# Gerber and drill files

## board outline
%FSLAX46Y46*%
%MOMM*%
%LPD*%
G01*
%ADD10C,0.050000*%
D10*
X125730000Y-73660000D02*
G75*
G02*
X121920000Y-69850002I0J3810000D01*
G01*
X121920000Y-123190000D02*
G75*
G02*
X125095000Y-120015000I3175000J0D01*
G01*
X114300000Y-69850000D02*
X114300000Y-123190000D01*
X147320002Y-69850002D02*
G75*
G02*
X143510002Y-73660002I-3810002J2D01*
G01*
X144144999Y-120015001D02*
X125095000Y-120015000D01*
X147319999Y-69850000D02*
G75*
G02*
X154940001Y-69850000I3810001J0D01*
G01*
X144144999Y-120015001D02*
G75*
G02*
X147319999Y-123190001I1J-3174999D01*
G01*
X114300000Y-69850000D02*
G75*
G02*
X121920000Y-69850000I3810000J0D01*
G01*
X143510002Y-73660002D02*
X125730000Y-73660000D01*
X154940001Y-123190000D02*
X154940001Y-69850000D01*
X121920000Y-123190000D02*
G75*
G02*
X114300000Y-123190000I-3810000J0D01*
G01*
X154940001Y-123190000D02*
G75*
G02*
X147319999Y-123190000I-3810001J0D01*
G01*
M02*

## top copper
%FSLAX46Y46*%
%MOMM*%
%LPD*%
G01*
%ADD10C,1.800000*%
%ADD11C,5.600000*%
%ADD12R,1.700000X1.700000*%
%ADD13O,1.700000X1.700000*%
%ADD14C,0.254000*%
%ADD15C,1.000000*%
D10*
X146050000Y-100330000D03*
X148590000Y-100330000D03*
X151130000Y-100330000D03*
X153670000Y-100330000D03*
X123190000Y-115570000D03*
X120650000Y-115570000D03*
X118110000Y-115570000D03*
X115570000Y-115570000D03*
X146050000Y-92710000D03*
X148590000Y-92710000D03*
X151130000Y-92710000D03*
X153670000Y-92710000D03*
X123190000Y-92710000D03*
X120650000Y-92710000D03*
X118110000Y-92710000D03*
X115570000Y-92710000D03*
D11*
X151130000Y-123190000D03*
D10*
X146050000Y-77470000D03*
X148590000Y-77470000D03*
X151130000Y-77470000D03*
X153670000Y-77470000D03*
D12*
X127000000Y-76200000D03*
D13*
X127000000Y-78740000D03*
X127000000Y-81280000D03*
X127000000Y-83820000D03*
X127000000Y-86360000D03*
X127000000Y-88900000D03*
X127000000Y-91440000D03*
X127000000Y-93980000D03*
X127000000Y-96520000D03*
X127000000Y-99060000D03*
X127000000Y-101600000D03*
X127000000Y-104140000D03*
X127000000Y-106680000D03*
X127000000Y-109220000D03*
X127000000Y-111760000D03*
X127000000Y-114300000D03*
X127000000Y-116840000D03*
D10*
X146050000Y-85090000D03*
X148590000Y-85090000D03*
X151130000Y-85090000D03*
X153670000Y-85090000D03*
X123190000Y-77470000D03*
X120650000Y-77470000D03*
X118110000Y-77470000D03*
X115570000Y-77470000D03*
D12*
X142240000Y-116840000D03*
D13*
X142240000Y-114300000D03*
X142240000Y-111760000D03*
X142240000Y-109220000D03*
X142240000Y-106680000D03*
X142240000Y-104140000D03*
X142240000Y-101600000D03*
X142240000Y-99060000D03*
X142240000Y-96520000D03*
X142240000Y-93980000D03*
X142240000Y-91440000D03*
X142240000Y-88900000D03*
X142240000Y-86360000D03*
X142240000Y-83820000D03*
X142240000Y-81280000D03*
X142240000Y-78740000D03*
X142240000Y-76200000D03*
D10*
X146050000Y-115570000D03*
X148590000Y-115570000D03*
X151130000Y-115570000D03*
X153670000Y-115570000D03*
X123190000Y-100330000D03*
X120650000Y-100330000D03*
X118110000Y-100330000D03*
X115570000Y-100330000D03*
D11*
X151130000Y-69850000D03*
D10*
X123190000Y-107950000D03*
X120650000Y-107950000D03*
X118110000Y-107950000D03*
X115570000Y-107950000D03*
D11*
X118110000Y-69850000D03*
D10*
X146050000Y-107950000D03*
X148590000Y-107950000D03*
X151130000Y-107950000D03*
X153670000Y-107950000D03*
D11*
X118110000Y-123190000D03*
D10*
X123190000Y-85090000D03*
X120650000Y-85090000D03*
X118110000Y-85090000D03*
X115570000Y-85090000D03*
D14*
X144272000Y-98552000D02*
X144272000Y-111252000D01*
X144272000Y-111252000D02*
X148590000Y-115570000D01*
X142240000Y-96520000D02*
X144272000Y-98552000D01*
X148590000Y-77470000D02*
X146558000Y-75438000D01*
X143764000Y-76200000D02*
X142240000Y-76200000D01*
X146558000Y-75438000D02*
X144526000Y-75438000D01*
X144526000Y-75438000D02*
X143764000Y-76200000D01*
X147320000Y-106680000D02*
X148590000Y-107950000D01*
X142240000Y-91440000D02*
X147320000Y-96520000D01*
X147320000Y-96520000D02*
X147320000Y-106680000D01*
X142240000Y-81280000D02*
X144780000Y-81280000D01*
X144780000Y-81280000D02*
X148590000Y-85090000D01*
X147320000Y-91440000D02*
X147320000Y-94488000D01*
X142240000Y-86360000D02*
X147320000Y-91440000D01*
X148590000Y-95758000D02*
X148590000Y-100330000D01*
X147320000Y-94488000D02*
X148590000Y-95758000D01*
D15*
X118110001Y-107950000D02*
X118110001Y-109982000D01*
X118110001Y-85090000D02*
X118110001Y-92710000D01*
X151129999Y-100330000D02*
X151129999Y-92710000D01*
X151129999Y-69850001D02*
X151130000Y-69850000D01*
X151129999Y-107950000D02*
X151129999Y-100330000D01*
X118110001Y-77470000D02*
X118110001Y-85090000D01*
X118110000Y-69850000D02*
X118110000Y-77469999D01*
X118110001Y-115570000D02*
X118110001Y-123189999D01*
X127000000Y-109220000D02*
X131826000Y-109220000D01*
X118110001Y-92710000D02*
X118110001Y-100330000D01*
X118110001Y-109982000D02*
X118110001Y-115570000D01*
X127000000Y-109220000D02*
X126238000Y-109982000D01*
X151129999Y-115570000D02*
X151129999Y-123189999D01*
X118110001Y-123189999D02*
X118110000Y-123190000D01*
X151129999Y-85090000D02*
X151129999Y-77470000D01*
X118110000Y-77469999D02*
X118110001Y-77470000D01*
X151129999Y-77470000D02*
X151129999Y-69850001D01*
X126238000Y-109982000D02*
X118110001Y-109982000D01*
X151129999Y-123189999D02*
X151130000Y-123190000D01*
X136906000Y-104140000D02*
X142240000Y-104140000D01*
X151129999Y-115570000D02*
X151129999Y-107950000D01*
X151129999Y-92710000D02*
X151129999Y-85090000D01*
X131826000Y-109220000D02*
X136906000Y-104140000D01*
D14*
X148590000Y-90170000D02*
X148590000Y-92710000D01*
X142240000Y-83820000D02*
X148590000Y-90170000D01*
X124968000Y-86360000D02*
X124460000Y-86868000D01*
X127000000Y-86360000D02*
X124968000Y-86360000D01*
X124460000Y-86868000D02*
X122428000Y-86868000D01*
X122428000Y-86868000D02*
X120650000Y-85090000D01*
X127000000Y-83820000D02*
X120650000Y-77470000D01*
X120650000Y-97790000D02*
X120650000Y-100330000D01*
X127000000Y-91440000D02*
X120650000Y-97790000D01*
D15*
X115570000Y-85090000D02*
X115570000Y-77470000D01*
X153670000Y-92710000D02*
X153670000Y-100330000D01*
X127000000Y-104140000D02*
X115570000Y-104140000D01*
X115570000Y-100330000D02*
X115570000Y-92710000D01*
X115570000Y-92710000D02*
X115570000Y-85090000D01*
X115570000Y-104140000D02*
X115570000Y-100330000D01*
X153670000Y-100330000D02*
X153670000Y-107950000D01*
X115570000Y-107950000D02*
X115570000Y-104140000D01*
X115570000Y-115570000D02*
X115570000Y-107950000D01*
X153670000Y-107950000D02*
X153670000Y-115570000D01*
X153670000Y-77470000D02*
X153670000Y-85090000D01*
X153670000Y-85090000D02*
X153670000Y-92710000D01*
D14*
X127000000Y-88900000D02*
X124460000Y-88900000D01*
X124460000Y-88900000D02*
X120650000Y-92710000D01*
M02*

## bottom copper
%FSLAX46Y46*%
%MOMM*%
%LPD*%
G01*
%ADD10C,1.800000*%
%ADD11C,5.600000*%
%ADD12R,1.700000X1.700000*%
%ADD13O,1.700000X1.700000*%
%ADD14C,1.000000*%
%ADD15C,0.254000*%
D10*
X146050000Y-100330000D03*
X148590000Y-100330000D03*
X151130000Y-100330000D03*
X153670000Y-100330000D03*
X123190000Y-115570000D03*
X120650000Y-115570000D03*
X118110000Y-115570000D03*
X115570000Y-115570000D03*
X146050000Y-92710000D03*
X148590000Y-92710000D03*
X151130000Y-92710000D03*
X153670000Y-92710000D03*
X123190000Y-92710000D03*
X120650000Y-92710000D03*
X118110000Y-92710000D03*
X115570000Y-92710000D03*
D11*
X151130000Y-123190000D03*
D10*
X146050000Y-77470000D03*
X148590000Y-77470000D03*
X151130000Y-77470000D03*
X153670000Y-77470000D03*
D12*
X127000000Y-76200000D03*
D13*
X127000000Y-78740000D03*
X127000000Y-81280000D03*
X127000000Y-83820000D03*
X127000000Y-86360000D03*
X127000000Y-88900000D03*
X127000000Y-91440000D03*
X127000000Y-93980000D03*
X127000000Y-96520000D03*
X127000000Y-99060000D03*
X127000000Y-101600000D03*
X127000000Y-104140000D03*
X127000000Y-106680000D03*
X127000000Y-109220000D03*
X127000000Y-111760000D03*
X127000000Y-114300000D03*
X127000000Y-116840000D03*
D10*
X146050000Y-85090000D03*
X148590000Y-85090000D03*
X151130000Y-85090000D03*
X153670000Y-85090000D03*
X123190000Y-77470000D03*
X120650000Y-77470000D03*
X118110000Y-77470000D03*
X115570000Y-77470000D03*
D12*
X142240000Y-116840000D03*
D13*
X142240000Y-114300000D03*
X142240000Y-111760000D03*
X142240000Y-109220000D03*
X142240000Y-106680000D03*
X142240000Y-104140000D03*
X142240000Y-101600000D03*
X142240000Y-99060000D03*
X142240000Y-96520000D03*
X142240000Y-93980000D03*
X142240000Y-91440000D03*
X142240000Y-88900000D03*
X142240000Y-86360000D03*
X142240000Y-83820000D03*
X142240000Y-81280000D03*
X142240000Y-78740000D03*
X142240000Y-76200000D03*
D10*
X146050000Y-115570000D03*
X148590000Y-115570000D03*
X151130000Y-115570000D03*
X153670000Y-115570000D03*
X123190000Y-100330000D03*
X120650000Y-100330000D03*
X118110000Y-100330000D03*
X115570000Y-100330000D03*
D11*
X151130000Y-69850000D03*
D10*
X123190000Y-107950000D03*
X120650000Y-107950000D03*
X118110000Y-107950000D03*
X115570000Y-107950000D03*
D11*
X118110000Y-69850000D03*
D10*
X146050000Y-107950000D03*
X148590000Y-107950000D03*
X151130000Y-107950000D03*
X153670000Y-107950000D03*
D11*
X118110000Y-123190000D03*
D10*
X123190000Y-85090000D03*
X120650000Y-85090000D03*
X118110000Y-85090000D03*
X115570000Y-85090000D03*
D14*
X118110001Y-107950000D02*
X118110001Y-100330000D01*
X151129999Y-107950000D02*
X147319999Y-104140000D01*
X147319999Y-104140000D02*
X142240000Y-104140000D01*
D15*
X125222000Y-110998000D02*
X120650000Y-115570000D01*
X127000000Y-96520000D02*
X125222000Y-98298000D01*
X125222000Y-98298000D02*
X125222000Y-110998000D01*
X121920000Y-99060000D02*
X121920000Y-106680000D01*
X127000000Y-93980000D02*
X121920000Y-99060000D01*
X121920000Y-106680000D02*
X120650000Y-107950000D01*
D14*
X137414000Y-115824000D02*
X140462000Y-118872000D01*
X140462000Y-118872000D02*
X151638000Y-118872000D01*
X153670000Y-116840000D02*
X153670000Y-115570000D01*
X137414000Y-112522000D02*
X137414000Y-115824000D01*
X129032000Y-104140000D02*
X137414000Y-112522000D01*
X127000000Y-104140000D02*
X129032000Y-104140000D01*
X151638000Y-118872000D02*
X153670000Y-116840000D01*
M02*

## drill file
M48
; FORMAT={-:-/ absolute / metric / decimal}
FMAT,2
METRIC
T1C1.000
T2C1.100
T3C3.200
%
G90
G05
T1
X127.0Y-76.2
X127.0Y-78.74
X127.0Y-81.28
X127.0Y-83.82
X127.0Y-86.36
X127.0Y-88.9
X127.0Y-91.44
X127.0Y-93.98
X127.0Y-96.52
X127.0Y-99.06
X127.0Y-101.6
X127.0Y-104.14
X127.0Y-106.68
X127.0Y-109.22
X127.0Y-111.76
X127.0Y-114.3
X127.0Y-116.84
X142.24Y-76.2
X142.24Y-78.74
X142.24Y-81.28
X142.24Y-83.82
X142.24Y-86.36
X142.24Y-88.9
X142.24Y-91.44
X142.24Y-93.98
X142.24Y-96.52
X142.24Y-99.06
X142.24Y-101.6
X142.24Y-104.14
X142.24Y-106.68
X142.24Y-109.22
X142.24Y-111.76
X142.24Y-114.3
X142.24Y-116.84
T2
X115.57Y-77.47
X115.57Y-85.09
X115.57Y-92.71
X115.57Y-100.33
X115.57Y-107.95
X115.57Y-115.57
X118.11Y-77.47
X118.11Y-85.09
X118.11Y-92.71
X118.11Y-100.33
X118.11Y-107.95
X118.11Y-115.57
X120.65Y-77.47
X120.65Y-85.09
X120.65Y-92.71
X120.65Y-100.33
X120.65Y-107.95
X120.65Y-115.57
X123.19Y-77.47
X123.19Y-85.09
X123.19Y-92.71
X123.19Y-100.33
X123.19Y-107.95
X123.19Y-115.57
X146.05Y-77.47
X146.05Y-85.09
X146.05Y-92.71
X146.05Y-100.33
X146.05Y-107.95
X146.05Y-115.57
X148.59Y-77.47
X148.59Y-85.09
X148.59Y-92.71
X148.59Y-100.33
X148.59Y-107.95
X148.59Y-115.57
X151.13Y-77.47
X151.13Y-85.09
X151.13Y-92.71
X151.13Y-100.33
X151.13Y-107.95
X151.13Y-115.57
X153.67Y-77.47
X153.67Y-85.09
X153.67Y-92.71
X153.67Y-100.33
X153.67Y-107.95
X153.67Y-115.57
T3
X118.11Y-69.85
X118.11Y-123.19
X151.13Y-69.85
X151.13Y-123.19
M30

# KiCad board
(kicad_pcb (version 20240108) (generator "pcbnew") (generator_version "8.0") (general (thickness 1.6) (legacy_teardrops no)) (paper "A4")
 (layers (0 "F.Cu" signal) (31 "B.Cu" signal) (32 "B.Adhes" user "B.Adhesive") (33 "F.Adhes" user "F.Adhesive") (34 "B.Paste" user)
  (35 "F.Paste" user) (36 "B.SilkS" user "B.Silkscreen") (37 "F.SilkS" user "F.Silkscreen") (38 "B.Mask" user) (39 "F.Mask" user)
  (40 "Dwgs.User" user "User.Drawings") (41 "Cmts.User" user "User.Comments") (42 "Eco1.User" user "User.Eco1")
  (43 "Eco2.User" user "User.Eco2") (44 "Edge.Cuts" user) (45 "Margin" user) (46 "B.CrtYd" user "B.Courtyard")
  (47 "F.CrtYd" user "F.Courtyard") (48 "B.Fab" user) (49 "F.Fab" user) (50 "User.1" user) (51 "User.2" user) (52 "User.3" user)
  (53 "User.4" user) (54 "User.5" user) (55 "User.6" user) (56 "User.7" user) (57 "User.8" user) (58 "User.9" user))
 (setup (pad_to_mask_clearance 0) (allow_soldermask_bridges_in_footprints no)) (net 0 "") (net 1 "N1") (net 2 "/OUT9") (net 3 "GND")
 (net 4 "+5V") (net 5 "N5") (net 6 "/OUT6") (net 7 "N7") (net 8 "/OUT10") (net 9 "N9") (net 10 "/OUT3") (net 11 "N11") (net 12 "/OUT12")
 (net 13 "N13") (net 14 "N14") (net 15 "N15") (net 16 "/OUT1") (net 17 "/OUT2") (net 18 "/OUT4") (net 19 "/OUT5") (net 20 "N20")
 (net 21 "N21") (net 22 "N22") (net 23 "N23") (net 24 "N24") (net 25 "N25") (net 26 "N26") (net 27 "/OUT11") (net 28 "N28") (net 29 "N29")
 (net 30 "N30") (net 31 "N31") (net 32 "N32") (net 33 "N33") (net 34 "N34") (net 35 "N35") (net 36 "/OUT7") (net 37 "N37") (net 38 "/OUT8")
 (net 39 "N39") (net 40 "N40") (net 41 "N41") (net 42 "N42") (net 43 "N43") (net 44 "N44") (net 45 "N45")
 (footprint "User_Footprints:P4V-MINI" (layer "F.Cu") (at 146.05 100.33)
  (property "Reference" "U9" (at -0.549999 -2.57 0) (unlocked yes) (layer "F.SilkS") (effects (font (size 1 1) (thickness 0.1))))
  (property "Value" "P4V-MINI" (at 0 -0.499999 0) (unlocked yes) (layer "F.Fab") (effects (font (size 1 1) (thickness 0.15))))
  (pad "1" thru_hole circle (at 0 0) (size 1.8 1.8) (drill 1.1) (layers "*.Cu" "*.Mask") (remove_unused_layers no) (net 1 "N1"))
  (pad "2" thru_hole circle (at 2.54 0) (size 1.8 1.8) (drill 1.1) (layers "*.Cu" "*.Mask") (remove_unused_layers no) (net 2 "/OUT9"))
  (pad "3" thru_hole circle (at 5.08 0) (size 1.8 1.8) (drill 1.1) (layers "*.Cu" "*.Mask") (remove_unused_layers no) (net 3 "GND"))
  (pad "4" thru_hole circle (at 7.62 0) (size 1.8 1.8) (drill 1.1) (layers "*.Cu" "*.Mask") (remove_unused_layers no) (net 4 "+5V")))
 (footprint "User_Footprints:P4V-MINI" (layer "F.Cu") (at 123.19 115.57 180)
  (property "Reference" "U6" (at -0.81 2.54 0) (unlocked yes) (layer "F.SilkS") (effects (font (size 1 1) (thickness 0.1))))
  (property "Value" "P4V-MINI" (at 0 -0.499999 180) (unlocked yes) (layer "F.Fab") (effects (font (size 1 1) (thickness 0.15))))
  (pad "1" thru_hole circle (at 0 0 180) (size 1.8 1.8) (drill 1.1) (layers "*.Cu" "*.Mask") (remove_unused_layers no) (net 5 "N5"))
  (pad "2" thru_hole circle (at 2.54 0 180) (size 1.8 1.8) (drill 1.1) (layers "*.Cu" "*.Mask") (remove_unused_layers no) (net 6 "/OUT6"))
  (pad "3" thru_hole circle (at 5.08 0 180) (size 1.8 1.8) (drill 1.1) (layers "*.Cu" "*.Mask") (remove_unused_layers no) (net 3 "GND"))
  (pad "4" thru_hole circle (at 7.62 0 180) (size 1.8 1.8) (drill 1.1) (layers "*.Cu" "*.Mask") (remove_unused_layers no) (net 4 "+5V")))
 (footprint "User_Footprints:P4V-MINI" (layer "F.Cu") (at 146.05 92.71)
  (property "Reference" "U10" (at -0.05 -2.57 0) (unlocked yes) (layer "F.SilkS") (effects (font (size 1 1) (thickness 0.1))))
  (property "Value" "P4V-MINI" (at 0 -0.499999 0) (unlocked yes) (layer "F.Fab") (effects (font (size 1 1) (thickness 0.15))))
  (pad "1" thru_hole circle (at 0 0) (size 1.8 1.8) (drill 1.1) (layers "*.Cu" "*.Mask") (remove_unused_layers no) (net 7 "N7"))
  (pad "2" thru_hole circle (at 2.54 0) (size 1.8 1.8) (drill 1.1) (layers "*.Cu" "*.Mask") (remove_unused_layers no) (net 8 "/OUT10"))
  (pad "3" thru_hole circle (at 5.08 0) (size 1.8 1.8) (drill 1.1) (layers "*.Cu" "*.Mask") (remove_unused_layers no) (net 3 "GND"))
  (pad "4" thru_hole circle (at 7.62 0) (size 1.8 1.8) (drill 1.1) (layers "*.Cu" "*.Mask") (remove_unused_layers no) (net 4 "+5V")))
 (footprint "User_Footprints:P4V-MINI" (layer "F.Cu") (at 123.19 92.71 180)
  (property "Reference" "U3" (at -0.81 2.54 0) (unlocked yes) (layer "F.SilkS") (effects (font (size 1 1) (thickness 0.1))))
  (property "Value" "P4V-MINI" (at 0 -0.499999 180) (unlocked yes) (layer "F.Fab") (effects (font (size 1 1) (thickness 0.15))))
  (pad "1" thru_hole circle (at 0 0 180) (size 1.8 1.8) (drill 1.1) (layers "*.Cu" "*.Mask") (remove_unused_layers no) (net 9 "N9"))
  (pad "2" thru_hole circle (at 2.54 0 180) (size 1.8 1.8) (drill 1.1) (layers "*.Cu" "*.Mask") (remove_unused_layers no) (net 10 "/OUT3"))
  (pad "3" thru_hole circle (at 5.08 0 180) (size 1.8 1.8) (drill 1.1) (layers "*.Cu" "*.Mask") (remove_unused_layers no) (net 3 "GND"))
  (pad "4" thru_hole circle (at 7.62 0 180) (size 1.8 1.8) (drill 1.1) (layers "*.Cu" "*.Mask") (remove_unused_layers no) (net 4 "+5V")))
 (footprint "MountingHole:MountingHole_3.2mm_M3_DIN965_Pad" (layer "F.Cu") (at 151.13 123.19)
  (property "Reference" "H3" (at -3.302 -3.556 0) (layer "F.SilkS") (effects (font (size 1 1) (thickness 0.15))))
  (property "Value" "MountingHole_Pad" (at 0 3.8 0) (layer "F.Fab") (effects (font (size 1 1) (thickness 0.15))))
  (pad "1" thru_hole circle (at 0 0) (size 5.6 5.6) (drill 3.2) (layers "*.Cu" "*.Mask") (remove_unused_layers no) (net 3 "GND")))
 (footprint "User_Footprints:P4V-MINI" (layer "F.Cu") (at 146.05 77.47)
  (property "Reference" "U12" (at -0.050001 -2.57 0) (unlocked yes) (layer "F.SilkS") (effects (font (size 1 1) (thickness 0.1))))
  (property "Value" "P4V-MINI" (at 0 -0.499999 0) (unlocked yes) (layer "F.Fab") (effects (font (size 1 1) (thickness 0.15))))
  (pad "1" thru_hole circle (at 0 0) (size 1.8 1.8) (drill 1.1) (layers "*.Cu" "*.Mask") (remove_unused_layers no) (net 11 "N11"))
  (pad "2" thru_hole circle (at 2.54 0) (size 1.8 1.8) (drill 1.1) (layers "*.Cu" "*.Mask") (remove_unused_layers no) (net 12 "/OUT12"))
  (pad "3" thru_hole circle (at 5.08 0) (size 1.8 1.8) (drill 1.1) (layers "*.Cu" "*.Mask") (remove_unused_layers no) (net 3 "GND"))
  (pad "4" thru_hole circle (at 7.62 0) (size 1.8 1.8) (drill 1.1) (layers "*.Cu" "*.Mask") (remove_unused_layers no) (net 4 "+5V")))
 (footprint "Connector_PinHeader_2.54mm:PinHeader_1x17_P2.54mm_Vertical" (layer "F.Cu") (at 127 76.2)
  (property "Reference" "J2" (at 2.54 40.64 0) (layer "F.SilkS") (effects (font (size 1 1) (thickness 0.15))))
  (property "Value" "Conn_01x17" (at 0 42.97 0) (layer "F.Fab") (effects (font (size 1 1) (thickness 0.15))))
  (pad "1" thru_hole rect (at 0 0) (size 1.7 1.7) (drill 1) (layers "*.Cu" "*.Mask") (remove_unused_layers no) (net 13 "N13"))
  (pad "2" thru_hole oval (at 0 2.54) (size 1.7 1.7) (drill 1) (layers "*.Cu" "*.Mask") (remove_unused_layers no) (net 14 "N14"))
  (pad "3" thru_hole oval (at 0 5.08) (size 1.7 1.7) (drill 1) (layers "*.Cu" "*.Mask") (remove_unused_layers no) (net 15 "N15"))
  (pad "4" thru_hole oval (at 0 7.62) (size 1.7 1.7) (drill 1) (layers "*.Cu" "*.Mask") (remove_unused_layers no) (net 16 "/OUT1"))
  (pad "5" thru_hole oval (at 0 10.16) (size 1.7 1.7) (drill 1) (layers "*.Cu" "*.Mask") (remove_unused_layers no) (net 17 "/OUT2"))
  (pad "6" thru_hole oval (at 0 12.7) (size 1.7 1.7) (drill 1) (layers "*.Cu" "*.Mask") (remove_unused_layers no) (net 10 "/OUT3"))
  (pad "7" thru_hole oval (at 0 15.24) (size 1.7 1.7) (drill 1) (layers "*.Cu" "*.Mask") (remove_unused_layers no) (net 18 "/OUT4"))
  (pad "8" thru_hole oval (at 0 17.78) (size 1.7 1.7) (drill 1) (layers "*.Cu" "*.Mask") (remove_unused_layers no) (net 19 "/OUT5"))
  (pad "9" thru_hole oval (at 0 20.32) (size 1.7 1.7) (drill 1) (layers "*.Cu" "*.Mask") (remove_unused_layers no) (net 6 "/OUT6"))
  (pad "10" thru_hole oval (at 0 22.86) (size 1.7 1.7) (drill 1) (layers "*.Cu" "*.Mask") (remove_unused_layers no) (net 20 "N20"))
  (pad "11" thru_hole oval (at 0 25.4) (size 1.7 1.7) (drill 1) (layers "*.Cu" "*.Mask") (remove_unused_layers no) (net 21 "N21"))
  (pad "12" thru_hole oval (at 0 27.94) (size 1.7 1.7) (drill 1) (layers "*.Cu" "*.Mask") (remove_unused_layers no) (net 4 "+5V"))
  (pad "13" thru_hole oval (at 0 30.48) (size 1.7 1.7) (drill 1) (layers "*.Cu" "*.Mask") (remove_unused_layers no) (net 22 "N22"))
  (pad "14" thru_hole oval (at 0 33.02) (size 1.7 1.7) (drill 1) (layers "*.Cu" "*.Mask") (remove_unused_layers no) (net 3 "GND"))
  (pad "15" thru_hole oval (at 0 35.56) (size 1.7 1.7) (drill 1) (layers "*.Cu" "*.Mask") (remove_unused_layers no) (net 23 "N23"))
  (pad "16" thru_hole oval (at 0 38.1) (size 1.7 1.7) (drill 1) (layers "*.Cu" "*.Mask") (remove_unused_layers no) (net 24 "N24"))
  (pad "17" thru_hole oval (at 0 40.64) (size 1.7 1.7) (drill 1) (layers "*.Cu" "*.Mask") (remove_unused_layers no) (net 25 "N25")))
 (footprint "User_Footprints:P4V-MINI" (layer "F.Cu") (at 146.05 85.09)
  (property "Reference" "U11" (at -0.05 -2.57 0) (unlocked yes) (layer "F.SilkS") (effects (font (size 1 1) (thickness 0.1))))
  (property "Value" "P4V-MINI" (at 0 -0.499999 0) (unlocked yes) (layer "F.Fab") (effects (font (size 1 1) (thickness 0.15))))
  (pad "1" thru_hole circle (at 0 0) (size 1.8 1.8) (drill 1.1) (layers "*.Cu" "*.Mask") (remove_unused_layers no) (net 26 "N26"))
  (pad "2" thru_hole circle (at 2.54 0) (size 1.8 1.8) (drill 1.1) (layers "*.Cu" "*.Mask") (remove_unused_layers no) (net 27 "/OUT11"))
  (pad "3" thru_hole circle (at 5.08 0) (size 1.8 1.8) (drill 1.1) (layers "*.Cu" "*.Mask") (remove_unused_layers no) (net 3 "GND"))
  (pad "4" thru_hole circle (at 7.62 0) (size 1.8 1.8) (drill 1.1) (layers "*.Cu" "*.Mask") (remove_unused_layers no) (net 4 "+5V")))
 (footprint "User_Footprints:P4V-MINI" (layer "F.Cu") (at 123.19 77.47 180)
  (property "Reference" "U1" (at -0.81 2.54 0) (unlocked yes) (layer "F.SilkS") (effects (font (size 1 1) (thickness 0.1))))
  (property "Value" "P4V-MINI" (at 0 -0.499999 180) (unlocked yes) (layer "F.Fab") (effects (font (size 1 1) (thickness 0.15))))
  (pad "1" thru_hole circle (at 0 0 180) (size 1.8 1.8) (drill 1.1) (layers "*.Cu" "*.Mask") (remove_unused_layers no) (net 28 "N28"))
  (pad "2" thru_hole circle (at 2.54 0 180) (size 1.8 1.8) (drill 1.1) (layers "*.Cu" "*.Mask") (remove_unused_layers no) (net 16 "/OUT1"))
  (pad "3" thru_hole circle (at 5.08 0 180) (size 1.8 1.8) (drill 1.1) (layers "*.Cu" "*.Mask") (remove_unused_layers no) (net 3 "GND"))
  (pad "4" thru_hole circle (at 7.62 0 180) (size 1.8 1.8) (drill 1.1) (layers "*.Cu" "*.Mask") (remove_unused_layers no) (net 4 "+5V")))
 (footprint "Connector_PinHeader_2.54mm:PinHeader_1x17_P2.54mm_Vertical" (layer "F.Cu") (at 142.24 116.84 180)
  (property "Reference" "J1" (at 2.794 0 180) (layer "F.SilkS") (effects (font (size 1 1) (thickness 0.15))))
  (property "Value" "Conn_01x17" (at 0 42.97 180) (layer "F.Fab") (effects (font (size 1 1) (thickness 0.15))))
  (pad "1" thru_hole rect (at 0 0 180) (size 1.7 1.7) (drill 1) (layers "*.Cu" "*.Mask") (remove_unused_layers no) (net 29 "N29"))
  (pad "2" thru_hole oval (at 0 2.54 180) (size 1.7 1.7) (drill 1) (layers "*.Cu" "*.Mask") (remove_unused_layers no) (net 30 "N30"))
  (pad "3" thru_hole oval (at 0 5.08 180) (size 1.7 1.7) (drill 1) (layers "*.Cu" "*.Mask") (remove_unused_layers no) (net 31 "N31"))
  (pad "4" thru_hole oval (at 0 7.62 180) (size 1.7 1.7) (drill 1) (layers "*.Cu" "*.Mask") (remove_unused_layers no) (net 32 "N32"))
  (pad "5" thru_hole oval (at 0 10.16 180) (size 1.7 1.7) (drill 1) (layers "*.Cu" "*.Mask") (remove_unused_layers no) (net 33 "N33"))
  (pad "6" thru_hole oval (at 0 12.7 180) (size 1.7 1.7) (drill 1) (layers "*.Cu" "*.Mask") (remove_unused_layers no) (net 3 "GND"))
  (pad "7" thru_hole oval (at 0 15.24 180) (size 1.7 1.7) (drill 1) (layers "*.Cu" "*.Mask") (remove_unused_layers no) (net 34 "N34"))
  (pad "8" thru_hole oval (at 0 17.78 180) (size 1.7 1.7) (drill 1) (layers "*.Cu" "*.Mask") (remove_unused_layers no) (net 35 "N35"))
  (pad "9" thru_hole oval (at 0 20.32 180) (size 1.7 1.7) (drill 1) (layers "*.Cu" "*.Mask") (remove_unused_layers no) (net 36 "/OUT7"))
  (pad "10" thru_hole oval (at 0 22.86 180) (size 1.7 1.7) (drill 1) (layers "*.Cu" "*.Mask") (remove_unused_layers no) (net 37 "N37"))
  (pad "11" thru_hole oval (at 0 25.4 180) (size 1.7 1.7) (drill 1) (layers "*.Cu" "*.Mask") (remove_unused_layers no) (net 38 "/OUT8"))
  (pad "12" thru_hole oval (at 0 27.94 180) (size 1.7 1.7) (drill 1) (layers "*.Cu" "*.Mask") (remove_unused_layers no) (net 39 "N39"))
  (pad "13" thru_hole oval (at 0 30.48 180) (size 1.7 1.7) (drill 1) (layers "*.Cu" "*.Mask") (remove_unused_layers no) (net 2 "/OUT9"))
  (pad "14" thru_hole oval (at 0 33.02 180) (size 1.7 1.7) (drill 1) (layers "*.Cu" "*.Mask") (remove_unused_layers no) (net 8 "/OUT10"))
  (pad "15" thru_hole oval (at 0 35.56 180) (size 1.7 1.7) (drill 1) (layers "*.Cu" "*.Mask") (remove_unused_layers no) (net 27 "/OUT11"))
  (pad "16" thru_hole oval (at 0 38.1 180) (size 1.7 1.7) (drill 1) (layers "*.Cu" "*.Mask") (remove_unused_layers no) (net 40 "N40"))
  (pad "17" thru_hole oval (at 0 40.64 180) (size 1.7 1.7) (drill 1) (layers "*.Cu" "*.Mask") (remove_unused_layers no) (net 12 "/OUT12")))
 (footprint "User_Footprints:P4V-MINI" (layer "F.Cu") (at 146.05 115.57)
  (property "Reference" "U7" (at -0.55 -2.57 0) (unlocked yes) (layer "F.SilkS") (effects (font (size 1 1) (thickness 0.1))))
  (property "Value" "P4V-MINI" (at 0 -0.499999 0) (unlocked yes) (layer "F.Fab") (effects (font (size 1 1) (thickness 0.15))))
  (pad "1" thru_hole circle (at 0 0) (size 1.8 1.8) (drill 1.1) (layers "*.Cu" "*.Mask") (remove_unused_layers no) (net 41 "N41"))
  (pad "2" thru_hole circle (at 2.54 0) (size 1.8 1.8) (drill 1.1) (layers "*.Cu" "*.Mask") (remove_unused_layers no) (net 36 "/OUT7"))
  (pad "3" thru_hole circle (at 5.08 0) (size 1.8 1.8) (drill 1.1) (layers "*.Cu" "*.Mask") (remove_unused_layers no) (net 3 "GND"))
  (pad "4" thru_hole circle (at 7.62 0) (size 1.8 1.8) (drill 1.1) (layers "*.Cu" "*.Mask") (remove_unused_layers no) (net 4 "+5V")))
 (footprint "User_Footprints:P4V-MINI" (layer "F.Cu") (at 123.19 100.33 180)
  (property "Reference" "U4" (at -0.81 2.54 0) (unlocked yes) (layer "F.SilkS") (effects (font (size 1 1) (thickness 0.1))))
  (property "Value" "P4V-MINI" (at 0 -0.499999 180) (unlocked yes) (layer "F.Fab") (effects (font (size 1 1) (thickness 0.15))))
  (pad "1" thru_hole circle (at 0 0 180) (size 1.8 1.8) (drill 1.1) (layers "*.Cu" "*.Mask") (remove_unused_layers no) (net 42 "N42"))
  (pad "2" thru_hole circle (at 2.54 0 180) (size 1.8 1.8) (drill 1.1) (layers "*.Cu" "*.Mask") (remove_unused_layers no) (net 18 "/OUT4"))
  (pad "3" thru_hole circle (at 5.08 0 180) (size 1.8 1.8) (drill 1.1) (layers "*.Cu" "*.Mask") (remove_unused_layers no) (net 3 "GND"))
  (pad "4" thru_hole circle (at 7.62 0 180) (size 1.8 1.8) (drill 1.1) (layers "*.Cu" "*.Mask") (remove_unused_layers no) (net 4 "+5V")))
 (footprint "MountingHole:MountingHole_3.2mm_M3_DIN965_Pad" (layer "F.Cu") (at 151.13 69.85)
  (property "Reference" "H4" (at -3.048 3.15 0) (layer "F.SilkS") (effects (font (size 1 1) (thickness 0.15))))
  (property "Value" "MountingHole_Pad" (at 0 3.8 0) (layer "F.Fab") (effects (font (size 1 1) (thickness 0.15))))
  (pad "1" thru_hole circle (at 0 0) (size 5.6 5.6) (drill 3.2) (layers "*.Cu" "*.Mask") (remove_unused_layers no) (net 3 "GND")))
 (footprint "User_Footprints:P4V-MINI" (layer "F.Cu") (at 123.19 107.95 180)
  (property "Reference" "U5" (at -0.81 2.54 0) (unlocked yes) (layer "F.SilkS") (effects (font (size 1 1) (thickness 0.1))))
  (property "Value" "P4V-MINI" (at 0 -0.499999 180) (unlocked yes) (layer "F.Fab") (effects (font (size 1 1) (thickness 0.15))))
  (pad "1" thru_hole circle (at 0 0 180) (size 1.8 1.8) (drill 1.1) (layers "*.Cu" "*.Mask") (remove_unused_layers no) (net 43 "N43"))
  (pad "2" thru_hole circle (at 2.54 0 180) (size 1.8 1.8) (drill 1.1) (layers "*.Cu" "*.Mask") (remove_unused_layers no) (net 19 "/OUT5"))
  (pad "3" thru_hole circle (at 5.08 0 180) (size 1.8 1.8) (drill 1.1) (layers "*.Cu" "*.Mask") (remove_unused_layers no) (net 3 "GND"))
  (pad "4" thru_hole circle (at 7.62 0 180) (size 1.8 1.8) (drill 1.1) (layers "*.Cu" "*.Mask") (remove_unused_layers no) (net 4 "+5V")))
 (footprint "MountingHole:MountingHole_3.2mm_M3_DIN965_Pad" (layer "F.Cu") (at 118.11 69.85)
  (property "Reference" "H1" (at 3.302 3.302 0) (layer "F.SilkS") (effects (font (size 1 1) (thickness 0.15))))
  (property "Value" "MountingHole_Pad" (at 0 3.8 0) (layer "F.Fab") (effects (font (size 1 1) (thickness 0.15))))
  (pad "1" thru_hole circle (at 0 0) (size 5.6 5.6) (drill 3.2) (layers "*.Cu" "*.Mask") (remove_unused_layers no) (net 3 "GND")))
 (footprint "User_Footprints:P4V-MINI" (layer "F.Cu") (at 146.05 107.95)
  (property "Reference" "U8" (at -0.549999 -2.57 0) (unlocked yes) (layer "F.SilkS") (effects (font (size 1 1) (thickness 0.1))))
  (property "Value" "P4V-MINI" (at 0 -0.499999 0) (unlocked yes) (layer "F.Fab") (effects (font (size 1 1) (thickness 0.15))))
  (pad "1" thru_hole circle (at 0 0) (size 1.8 1.8) (drill 1.1) (layers "*.Cu" "*.Mask") (remove_unused_layers no) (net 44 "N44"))
  (pad "2" thru_hole circle (at 2.54 0) (size 1.8 1.8) (drill 1.1) (layers "*.Cu" "*.Mask") (remove_unused_layers no) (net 38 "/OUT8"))
  (pad "3" thru_hole circle (at 5.08 0) (size 1.8 1.8) (drill 1.1) (layers "*.Cu" "*.Mask") (remove_unused_layers no) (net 3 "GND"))
  (pad "4" thru_hole circle (at 7.62 0) (size 1.8 1.8) (drill 1.1) (layers "*.Cu" "*.Mask") (remove_unused_layers no) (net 4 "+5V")))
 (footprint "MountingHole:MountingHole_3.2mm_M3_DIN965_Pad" (layer "F.Cu") (at 118.11 123.19)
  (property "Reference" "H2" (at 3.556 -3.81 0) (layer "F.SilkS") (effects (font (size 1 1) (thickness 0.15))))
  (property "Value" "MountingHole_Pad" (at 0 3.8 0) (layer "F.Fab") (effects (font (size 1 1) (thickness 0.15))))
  (pad "1" thru_hole circle (at 0 0) (size 5.6 5.6) (drill 3.2) (layers "*.Cu" "*.Mask") (remove_unused_layers no) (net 3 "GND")))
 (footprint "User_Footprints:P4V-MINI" (layer "F.Cu") (at 123.19 85.09 180)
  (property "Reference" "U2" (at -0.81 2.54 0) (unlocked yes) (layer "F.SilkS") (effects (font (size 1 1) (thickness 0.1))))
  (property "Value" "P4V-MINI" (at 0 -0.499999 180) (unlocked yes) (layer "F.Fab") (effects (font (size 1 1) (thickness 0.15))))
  (pad "1" thru_hole circle (at 0 0 180) (size 1.8 1.8) (drill 1.1) (layers "*.Cu" "*.Mask") (remove_unused_layers no) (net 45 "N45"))
  (pad "2" thru_hole circle (at 2.54 0 180) (size 1.8 1.8) (drill 1.1) (layers "*.Cu" "*.Mask") (remove_unused_layers no) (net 17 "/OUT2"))
  (pad "3" thru_hole circle (at 5.08 0 180) (size 1.8 1.8) (drill 1.1) (layers "*.Cu" "*.Mask") (remove_unused_layers no) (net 3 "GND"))
  (pad "4" thru_hole circle (at 7.62 0 180) (size 1.8 1.8) (drill 1.1) (layers "*.Cu" "*.Mask") (remove_unused_layers no) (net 4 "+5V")))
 (gr_arc (start 125.73 73.66) (mid 123.035924 72.544078) (end 121.92 69.850002) (stroke (width 0.05) (type default)) (layer "Edge.Cuts"))
 (gr_arc (start 121.92 123.19) (mid 122.849936 120.944936) (end 125.095 120.015) (stroke (width 0.05) (type default)) (layer "Edge.Cuts"))
 (gr_line (start 114.3 69.85) (end 114.3 123.19) (stroke (width 0.05) (type default)) (layer "Edge.Cuts"))
 (gr_arc (start 147.320002 69.850002) (mid 146.204078 72.544078) (end 143.510002 73.660002) (stroke (width 0.05) (type default))
  (layer "Edge.Cuts"))
 (gr_line (start 144.144999 120.015001) (end 125.095 120.015) (stroke (width 0.05) (type default)) (layer "Edge.Cuts"))
 (gr_arc (start 147.319999 69.85) (mid 151.13 66.039999) (end 154.940001 69.85) (stroke (width 0.05) (type default)) (layer "Edge.Cuts"))
 (gr_arc (start 144.144999 120.015001) (mid 146.390063 120.944937) (end 147.319999 123.190001) (stroke (width 0.05) (type default))
  (layer "Edge.Cuts"))
 (gr_arc (start 114.3 69.85) (mid 118.11 66.04) (end 121.92 69.85) (stroke (width 0.05) (type default)) (layer "Edge.Cuts"))
 (gr_line (start 143.510002 73.660002) (end 125.73 73.66) (stroke (width 0.05) (type default)) (layer "Edge.Cuts"))
 (gr_line (start 154.940001 123.19) (end 154.940001 69.85) (stroke (width 0.05) (type default)) (layer "Edge.Cuts"))
 (gr_arc (start 121.92 123.19) (mid 118.11 127) (end 114.3 123.19) (stroke (width 0.05) (type default)) (layer "Edge.Cuts"))
 (gr_arc (start 154.940001 123.19) (mid 151.13 127.000001) (end 147.319999 123.19) (stroke (width 0.05) (type default)) (layer "Edge.Cuts"))
 (segment (start 144.272 98.552) (end 144.272 111.252) (width 0.254) (layer "F.Cu") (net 36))
 (segment (start 144.272 111.252) (end 148.59 115.57) (width 0.254) (layer "F.Cu") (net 36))
 (segment (start 142.24 96.52) (end 144.272 98.552) (width 0.254) (layer "F.Cu") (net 36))
 (segment (start 148.59 77.47) (end 146.558 75.438) (width 0.254) (layer "F.Cu") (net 12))
 (segment (start 143.764 76.2) (end 142.24 76.2) (width 0.254) (layer "F.Cu") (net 12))
 (segment (start 146.558 75.438) (end 144.526 75.438) (width 0.254) (layer "F.Cu") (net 12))
 (segment (start 144.526 75.438) (end 143.764 76.2) (width 0.254) (layer "F.Cu") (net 12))
 (segment (start 147.32 106.68) (end 148.59 107.95) (width 0.254) (layer "F.Cu") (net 38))
 (segment (start 142.24 91.44) (end 147.32 96.52) (width 0.254) (layer "F.Cu") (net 38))
 (segment (start 147.32 96.52) (end 147.32 106.68) (width 0.254) (layer "F.Cu") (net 38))
 (segment (start 142.24 81.28) (end 144.78 81.28) (width 0.254) (layer "F.Cu") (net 27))
 (segment (start 144.78 81.28) (end 148.59 85.09) (width 0.254) (layer "F.Cu") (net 27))
 (segment (start 147.32 91.44) (end 147.32 94.488) (width 0.254) (layer "F.Cu") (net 2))
 (segment (start 142.24 86.36) (end 147.32 91.44) (width 0.254) (layer "F.Cu") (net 2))
 (segment (start 148.59 95.758) (end 148.59 100.33) (width 0.254) (layer "F.Cu") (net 2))
 (segment (start 147.32 94.488) (end 148.59 95.758) (width 0.254) (layer "F.Cu") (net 2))
 (segment (start 118.110001 107.95) (end 118.110001 109.982) (width 1) (layer "F.Cu") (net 3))
 (segment (start 118.110001 85.09) (end 118.110001 92.71) (width 1) (layer "F.Cu") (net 3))
 (segment (start 151.129999 100.33) (end 151.129999 92.71) (width 1) (layer "F.Cu") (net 3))
 (segment (start 151.129999 69.850001) (end 151.13 69.85) (width 1) (layer "F.Cu") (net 3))
 (segment (start 151.129999 107.95) (end 151.129999 100.33) (width 1) (layer "F.Cu") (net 3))
 (segment (start 118.110001 77.47) (end 118.110001 85.09) (width 1) (layer "F.Cu") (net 3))
 (segment (start 118.11 69.85) (end 118.11 77.469999) (width 1) (layer "F.Cu") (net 3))
 (segment (start 118.110001 115.57) (end 118.110001 123.189999) (width 1) (layer "F.Cu") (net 3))
 (segment (start 127 109.22) (end 131.826 109.22) (width 1) (layer "F.Cu") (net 3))
 (segment (start 118.110001 92.71) (end 118.110001 100.33) (width 1) (layer "F.Cu") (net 3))
 (segment (start 118.110001 109.982) (end 118.110001 115.57) (width 1) (layer "F.Cu") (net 3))
 (segment (start 127 109.22) (end 126.238 109.982) (width 1) (layer "F.Cu") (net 3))
 (segment (start 151.129999 115.57) (end 151.129999 123.189999) (width 1) (layer "F.Cu") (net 3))
 (segment (start 118.110001 123.189999) (end 118.11 123.19) (width 1) (layer "F.Cu") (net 3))
 (segment (start 151.129999 85.09) (end 151.129999 77.47) (width 1) (layer "F.Cu") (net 3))
 (segment (start 118.11 77.469999) (end 118.110001 77.47) (width 1) (layer "F.Cu") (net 3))
 (segment (start 151.129999 77.47) (end 151.129999 69.850001) (width 1) (layer "F.Cu") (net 3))
 (segment (start 126.238 109.982) (end 118.110001 109.982) (width 1) (layer "F.Cu") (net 3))
 (segment (start 151.129999 123.189999) (end 151.13 123.19) (width 1) (layer "F.Cu") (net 3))
 (segment (start 136.906 104.14) (end 142.24 104.14) (width 1) (layer "F.Cu") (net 3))
 (segment (start 151.129999 115.57) (end 151.129999 107.95) (width 1) (layer "F.Cu") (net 3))
 (segment (start 151.129999 92.71) (end 151.129999 85.09) (width 1) (layer "F.Cu") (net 3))
 (segment (start 131.826 109.22) (end 136.906 104.14) (width 1) (layer "F.Cu") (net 3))
 (segment (start 118.110001 107.95) (end 118.110001 100.33) (width 1) (layer "B.Cu") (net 3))
 (segment (start 151.129999 107.95) (end 147.319999 104.14) (width 1) (layer "B.Cu") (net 3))
 (segment (start 147.319999 104.14) (end 142.24 104.14) (width 1) (layer "B.Cu") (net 3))
 (segment (start 148.59 90.17) (end 148.59 92.71) (width 0.254) (layer "F.Cu") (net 8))
 (segment (start 142.24 83.82) (end 148.59 90.17) (width 0.254) (layer "F.Cu") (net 8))
 (segment (start 124.968 86.36) (end 124.46 86.868) (width 0.254) (layer "F.Cu") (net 17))
 (segment (start 127 86.36) (end 124.968 86.36) (width 0.254) (layer "F.Cu") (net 17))
 (segment (start 124.46 86.868) (end 122.428 86.868) (width 0.254) (layer "F.Cu") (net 17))
 (segment (start 122.428 86.868) (end 120.65 85.09) (width 0.254) (layer "F.Cu") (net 17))
 (segment (start 127 83.82) (end 120.65 77.47) (width 0.254) (layer "F.Cu") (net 16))
 (segment (start 125.222 110.998) (end 120.65 115.57) (width 0.254) (layer "B.Cu") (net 6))
 (segment (start 127 96.52) (end 125.222 98.298) (width 0.254) (layer "B.Cu") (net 6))
 (segment (start 125.222 98.298) (end 125.222 110.998) (width 0.254) (layer "B.Cu") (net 6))
 (segment (start 120.65 97.79) (end 120.65 100.33) (width 0.254) (layer "F.Cu") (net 18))
 (segment (start 127 91.44) (end 120.65 97.79) (width 0.254) (layer "F.Cu") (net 18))
 (segment (start 121.92 99.06) (end 121.92 106.68) (width 0.254) (layer "B.Cu") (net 19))
 (segment (start 127 93.98) (end 121.92 99.06) (width 0.254) (layer "B.Cu") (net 19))
 (segment (start 121.92 106.68) (end 120.65 107.95) (width 0.254) (layer "B.Cu") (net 19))
 (segment (start 115.57 85.09) (end 115.57 77.47) (width 1) (layer "F.Cu") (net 4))
 (segment (start 153.67 92.71) (end 153.67 100.33) (width 1) (layer "F.Cu") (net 4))
 (segment (start 127 104.14) (end 115.57 104.14) (width 1) (layer "F.Cu") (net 4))
 (segment (start 115.57 100.33) (end 115.57 92.71) (width 1) (layer "F.Cu") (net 4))
 (segment (start 115.57 92.71) (end 115.57 85.09) (width 1) (layer "F.Cu") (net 4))
 (segment (start 115.57 104.14) (end 115.57 100.33) (width 1) (layer "F.Cu") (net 4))
 (segment (start 153.67 100.33) (end 153.67 107.95) (width 1) (layer "F.Cu") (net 4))
 (segment (start 115.57 107.95) (end 115.57 104.14) (width 1) (layer "F.Cu") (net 4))
 (segment (start 115.57 115.57) (end 115.57 107.95) (width 1) (layer "F.Cu") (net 4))
 (segment (start 153.67 107.95) (end 153.67 115.57) (width 1) (layer "F.Cu") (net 4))
 (segment (start 153.67 77.47) (end 153.67 85.09) (width 1) (layer "F.Cu") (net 4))
 (segment (start 153.67 85.09) (end 153.67 92.71) (width 1) (layer "F.Cu") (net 4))
 (segment (start 137.414 115.824) (end 140.462 118.872) (width 1) (layer "B.Cu") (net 4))
 (segment (start 140.462 118.872) (end 151.638 118.872) (width 1) (layer "B.Cu") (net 4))
 (segment (start 153.67 116.84) (end 153.67 115.57) (width 1) (layer "B.Cu") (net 4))
 (segment (start 137.414 112.522) (end 137.414 115.824) (width 1) (layer "B.Cu") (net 4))
 (segment (start 129.032 104.14) (end 137.414 112.522) (width 1) (layer "B.Cu") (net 4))
 (segment (start 127 104.14) (end 129.032 104.14) (width 1) (layer "B.Cu") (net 4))
 (segment (start 151.638 118.872) (end 153.67 116.84) (width 1) (layer "B.Cu") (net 4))
 (segment (start 127 88.9) (end 124.46 88.9) (width 0.254) (layer "F.Cu") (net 10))
 (segment (start 124.46 88.9) (end 120.65 92.71) (width 0.254) (layer "F.Cu") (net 10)))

